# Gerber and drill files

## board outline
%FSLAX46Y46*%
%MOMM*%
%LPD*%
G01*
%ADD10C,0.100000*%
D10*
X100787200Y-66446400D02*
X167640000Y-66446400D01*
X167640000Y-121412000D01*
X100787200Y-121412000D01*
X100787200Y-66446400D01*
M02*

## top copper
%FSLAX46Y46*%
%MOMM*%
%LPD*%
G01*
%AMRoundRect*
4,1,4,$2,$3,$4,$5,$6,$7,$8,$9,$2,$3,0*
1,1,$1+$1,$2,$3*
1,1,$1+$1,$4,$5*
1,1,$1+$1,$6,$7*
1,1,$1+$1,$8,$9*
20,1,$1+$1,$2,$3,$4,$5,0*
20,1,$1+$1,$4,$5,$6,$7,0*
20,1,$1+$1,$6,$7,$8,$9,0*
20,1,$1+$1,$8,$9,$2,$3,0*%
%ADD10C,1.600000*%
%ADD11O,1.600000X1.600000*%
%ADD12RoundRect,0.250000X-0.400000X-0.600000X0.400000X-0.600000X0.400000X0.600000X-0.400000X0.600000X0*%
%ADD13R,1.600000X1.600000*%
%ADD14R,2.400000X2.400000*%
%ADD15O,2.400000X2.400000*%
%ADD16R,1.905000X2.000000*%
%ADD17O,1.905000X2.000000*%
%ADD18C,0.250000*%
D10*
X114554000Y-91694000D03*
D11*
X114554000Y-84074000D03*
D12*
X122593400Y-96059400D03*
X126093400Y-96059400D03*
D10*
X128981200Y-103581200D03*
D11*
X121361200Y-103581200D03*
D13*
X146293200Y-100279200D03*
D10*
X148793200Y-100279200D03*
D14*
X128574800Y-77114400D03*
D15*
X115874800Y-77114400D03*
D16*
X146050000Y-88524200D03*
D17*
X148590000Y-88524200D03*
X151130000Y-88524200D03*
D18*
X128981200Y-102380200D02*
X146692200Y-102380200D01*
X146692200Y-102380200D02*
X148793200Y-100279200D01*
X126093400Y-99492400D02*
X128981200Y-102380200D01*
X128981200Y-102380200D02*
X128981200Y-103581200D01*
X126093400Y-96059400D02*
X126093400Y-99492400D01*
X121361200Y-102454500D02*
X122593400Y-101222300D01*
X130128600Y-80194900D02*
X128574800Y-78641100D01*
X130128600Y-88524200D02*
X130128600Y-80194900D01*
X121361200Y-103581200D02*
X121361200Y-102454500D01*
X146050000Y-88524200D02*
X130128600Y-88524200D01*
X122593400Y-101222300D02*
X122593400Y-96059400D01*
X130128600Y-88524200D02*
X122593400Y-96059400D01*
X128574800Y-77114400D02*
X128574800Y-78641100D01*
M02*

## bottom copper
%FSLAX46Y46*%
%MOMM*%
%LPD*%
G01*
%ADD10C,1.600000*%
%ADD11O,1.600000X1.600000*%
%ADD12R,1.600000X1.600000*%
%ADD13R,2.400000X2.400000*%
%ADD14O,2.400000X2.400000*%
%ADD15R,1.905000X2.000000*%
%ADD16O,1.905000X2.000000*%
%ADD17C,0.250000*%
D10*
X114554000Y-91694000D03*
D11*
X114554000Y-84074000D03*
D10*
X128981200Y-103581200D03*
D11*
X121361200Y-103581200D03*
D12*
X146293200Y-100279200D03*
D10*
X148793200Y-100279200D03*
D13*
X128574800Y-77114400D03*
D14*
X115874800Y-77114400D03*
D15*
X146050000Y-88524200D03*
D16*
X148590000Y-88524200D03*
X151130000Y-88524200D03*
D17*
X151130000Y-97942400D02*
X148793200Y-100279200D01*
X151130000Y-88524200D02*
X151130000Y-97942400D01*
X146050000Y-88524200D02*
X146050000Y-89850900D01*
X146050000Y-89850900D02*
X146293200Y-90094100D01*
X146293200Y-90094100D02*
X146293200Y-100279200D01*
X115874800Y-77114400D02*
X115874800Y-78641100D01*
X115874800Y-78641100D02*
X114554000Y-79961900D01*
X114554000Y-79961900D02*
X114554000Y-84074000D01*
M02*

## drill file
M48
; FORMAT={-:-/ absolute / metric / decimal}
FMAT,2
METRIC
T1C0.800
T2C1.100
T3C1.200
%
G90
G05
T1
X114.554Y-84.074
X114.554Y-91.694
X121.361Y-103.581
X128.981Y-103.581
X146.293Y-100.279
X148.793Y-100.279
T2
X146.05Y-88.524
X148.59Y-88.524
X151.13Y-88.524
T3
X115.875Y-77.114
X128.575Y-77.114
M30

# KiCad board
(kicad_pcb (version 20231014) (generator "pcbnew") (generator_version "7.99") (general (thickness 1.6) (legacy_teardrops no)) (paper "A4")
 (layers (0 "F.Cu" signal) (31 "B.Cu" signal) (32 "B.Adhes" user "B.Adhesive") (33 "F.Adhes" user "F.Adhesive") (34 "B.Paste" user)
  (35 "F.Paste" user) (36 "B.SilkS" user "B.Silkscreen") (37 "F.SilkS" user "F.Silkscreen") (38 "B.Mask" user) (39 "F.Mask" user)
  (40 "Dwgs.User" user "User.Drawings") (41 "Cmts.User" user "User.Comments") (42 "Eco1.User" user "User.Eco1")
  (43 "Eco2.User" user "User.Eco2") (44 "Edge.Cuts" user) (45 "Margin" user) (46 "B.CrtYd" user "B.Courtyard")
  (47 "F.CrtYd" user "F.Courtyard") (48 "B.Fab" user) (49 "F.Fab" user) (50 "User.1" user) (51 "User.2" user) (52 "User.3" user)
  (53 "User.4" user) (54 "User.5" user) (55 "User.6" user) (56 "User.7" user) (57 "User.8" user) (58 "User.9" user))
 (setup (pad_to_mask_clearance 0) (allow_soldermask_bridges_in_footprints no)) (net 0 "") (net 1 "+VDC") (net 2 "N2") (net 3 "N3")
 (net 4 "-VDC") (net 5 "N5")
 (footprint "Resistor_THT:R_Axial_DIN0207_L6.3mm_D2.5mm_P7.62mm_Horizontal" (layer "F.Cu") (at 114.554 91.694 90)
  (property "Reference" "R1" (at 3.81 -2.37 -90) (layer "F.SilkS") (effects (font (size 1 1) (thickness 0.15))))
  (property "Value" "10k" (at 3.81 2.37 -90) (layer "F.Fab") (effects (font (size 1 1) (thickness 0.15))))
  (pad "1" thru_hole circle (at 0 0 90) (size 1.6 1.6) (drill 0.8) (layers "*.Cu" "*.Mask") (remove_unused_layers no) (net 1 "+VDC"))
  (pad "2" thru_hole oval (at 7.62 0 90) (size 1.6 1.6) (drill 0.8) (layers "*.Cu" "*.Mask") (remove_unused_layers no) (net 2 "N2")))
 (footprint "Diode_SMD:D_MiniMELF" (layer "F.Cu") (at 124.3434 96.0594)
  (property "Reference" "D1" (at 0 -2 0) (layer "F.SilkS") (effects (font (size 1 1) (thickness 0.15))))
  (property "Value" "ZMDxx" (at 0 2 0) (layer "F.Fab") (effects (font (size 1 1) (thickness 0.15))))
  (pad "1" smd roundrect (at -1.75 0) (size 1.3 1.7) (layers "F.Cu" "F.Paste" "F.Mask") (roundrect_rratio 0.1923076923) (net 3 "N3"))
  (pad "2" smd roundrect (at 1.75 0) (size 1.3 1.7) (layers "F.Cu" "F.Paste" "F.Mask") (roundrect_rratio 0.1923076923) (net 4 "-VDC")))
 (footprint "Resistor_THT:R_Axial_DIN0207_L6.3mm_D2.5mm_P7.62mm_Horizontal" (layer "F.Cu") (at 128.9812 103.5812 180)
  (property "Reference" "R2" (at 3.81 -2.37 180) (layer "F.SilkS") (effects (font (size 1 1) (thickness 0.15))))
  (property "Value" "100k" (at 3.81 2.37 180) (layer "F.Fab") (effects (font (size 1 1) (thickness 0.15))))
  (pad "1" thru_hole circle (at 0 0 180) (size 1.6 1.6) (drill 0.8) (layers "*.Cu" "*.Mask") (remove_unused_layers no) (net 4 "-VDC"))
  (pad "2" thru_hole oval (at 7.62 0 180) (size 1.6 1.6) (drill 0.8) (layers "*.Cu" "*.Mask") (remove_unused_layers no) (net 3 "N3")))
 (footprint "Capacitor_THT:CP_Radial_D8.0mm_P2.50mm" (layer "F.Cu") (at 146.2932 100.2792)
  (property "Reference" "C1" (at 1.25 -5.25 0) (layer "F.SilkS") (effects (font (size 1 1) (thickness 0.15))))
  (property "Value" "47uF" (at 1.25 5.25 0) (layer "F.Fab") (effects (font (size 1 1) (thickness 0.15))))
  (pad "1" thru_hole rect (at 0 0) (size 1.6 1.6) (drill 0.8) (layers "*.Cu" "*.Mask") (remove_unused_layers no) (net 3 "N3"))
  (pad "2" thru_hole circle (at 2.5 0) (size 1.6 1.6) (drill 0.8) (layers "*.Cu" "*.Mask") (remove_unused_layers no) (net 4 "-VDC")))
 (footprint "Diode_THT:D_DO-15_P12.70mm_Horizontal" (layer "F.Cu") (at 128.5748 77.1144 180)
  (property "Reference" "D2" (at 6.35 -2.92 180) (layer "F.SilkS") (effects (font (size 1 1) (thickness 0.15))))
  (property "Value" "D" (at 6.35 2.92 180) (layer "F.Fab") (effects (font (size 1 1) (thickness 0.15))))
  (pad "1" thru_hole rect (at 0 0 180) (size 2.4 2.4) (drill 1.2) (layers "*.Cu" "*.Mask") (remove_unused_layers no) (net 3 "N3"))
  (pad "2" thru_hole oval (at 12.7 0 180) (size 2.4 2.4) (drill 1.2) (layers "*.Cu" "*.Mask") (remove_unused_layers no) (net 2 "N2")))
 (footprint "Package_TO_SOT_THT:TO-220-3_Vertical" (layer "F.Cu") (at 146.05 88.5242)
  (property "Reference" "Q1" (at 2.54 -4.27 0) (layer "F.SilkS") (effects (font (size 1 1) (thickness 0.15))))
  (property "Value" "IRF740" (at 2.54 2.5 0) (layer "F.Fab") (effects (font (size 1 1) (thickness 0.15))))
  (pad "1" thru_hole rect (at 0 0) (size 1.905 2) (drill 1.1) (layers "*.Cu" "*.Mask") (remove_unused_layers no) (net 3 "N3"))
  (pad "2" thru_hole oval (at 2.54 0) (size 1.905 2) (drill 1.1) (layers "*.Cu" "*.Mask") (remove_unused_layers no) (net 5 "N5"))
  (pad "3" thru_hole oval (at 5.08 0) (size 1.905 2) (drill 1.1) (layers "*.Cu" "*.Mask") (remove_unused_layers no) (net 4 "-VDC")))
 (gr_rect (start 100.7872 66.4464) (end 167.64 121.412) (stroke (width 0.1) (type default)) (fill none) (layer "Edge.Cuts"))
 (segment (start 128.9812 102.3802) (end 146.6922 102.3802) (width 0.25) (layer "F.Cu") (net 4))
 (segment (start 146.6922 102.3802) (end 148.7932 100.2792) (width 0.25) (layer "F.Cu") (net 4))
 (segment (start 126.0934 99.4924) (end 128.9812 102.3802) (width 0.25) (layer "F.Cu") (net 4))
 (segment (start 128.9812 102.3802) (end 128.9812 103.5812) (width 0.25) (layer "F.Cu") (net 4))
 (segment (start 126.0934 96.0594) (end 126.0934 99.4924) (width 0.25) (layer "F.Cu") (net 4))
 (segment (start 151.13 97.9424) (end 148.7932 100.2792) (width 0.25) (layer "B.Cu") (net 4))
 (segment (start 151.13 88.5242) (end 151.13 97.9424) (width 0.25) (layer "B.Cu") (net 4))
 (segment (start 121.3612 102.4545) (end 122.5934 101.2223) (width 0.25) (layer "F.Cu") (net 3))
 (segment (start 130.1286 80.1949) (end 128.5748 78.6411) (width 0.25) (layer "F.Cu") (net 3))
 (segment (start 130.1286 88.5242) (end 130.1286 80.1949) (width 0.25) (layer "F.Cu") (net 3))
 (segment (start 121.3612 103.5812) (end 121.3612 102.4545) (width 0.25) (layer "F.Cu") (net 3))
 (segment (start 146.05 88.5242) (end 130.1286 88.5242) (width 0.25) (layer "F.Cu") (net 3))
 (segment (start 122.5934 101.2223) (end 122.5934 96.0594) (width 0.25) (layer "F.Cu") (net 3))
 (segment (start 130.1286 88.5242) (end 122.5934 96.0594) (width 0.25) (layer "F.Cu") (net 3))
 (segment (start 128.5748 77.1144) (end 128.5748 78.6411) (width 0.25) (layer "F.Cu") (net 3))
 (segment (start 146.05 88.5242) (end 146.05 89.8509) (width 0.25) (layer "B.Cu") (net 3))
 (segment (start 146.05 89.8509) (end 146.2932 90.0941) (width 0.25) (layer "B.Cu") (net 3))
 (segment (start 146.2932 90.0941) (end 146.2932 100.2792) (width 0.25) (layer "B.Cu") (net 3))
 (segment (start 115.8748 77.1144) (end 115.8748 78.6411) (width 0.25) (layer "B.Cu") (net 2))
 (segment (start 115.8748 78.6411) (end 114.554 79.9619) (width 0.25) (layer "B.Cu") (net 2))
 (segment (start 114.554 79.9619) (end 114.554 84.074) (width 0.25) (layer "B.Cu") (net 2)))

